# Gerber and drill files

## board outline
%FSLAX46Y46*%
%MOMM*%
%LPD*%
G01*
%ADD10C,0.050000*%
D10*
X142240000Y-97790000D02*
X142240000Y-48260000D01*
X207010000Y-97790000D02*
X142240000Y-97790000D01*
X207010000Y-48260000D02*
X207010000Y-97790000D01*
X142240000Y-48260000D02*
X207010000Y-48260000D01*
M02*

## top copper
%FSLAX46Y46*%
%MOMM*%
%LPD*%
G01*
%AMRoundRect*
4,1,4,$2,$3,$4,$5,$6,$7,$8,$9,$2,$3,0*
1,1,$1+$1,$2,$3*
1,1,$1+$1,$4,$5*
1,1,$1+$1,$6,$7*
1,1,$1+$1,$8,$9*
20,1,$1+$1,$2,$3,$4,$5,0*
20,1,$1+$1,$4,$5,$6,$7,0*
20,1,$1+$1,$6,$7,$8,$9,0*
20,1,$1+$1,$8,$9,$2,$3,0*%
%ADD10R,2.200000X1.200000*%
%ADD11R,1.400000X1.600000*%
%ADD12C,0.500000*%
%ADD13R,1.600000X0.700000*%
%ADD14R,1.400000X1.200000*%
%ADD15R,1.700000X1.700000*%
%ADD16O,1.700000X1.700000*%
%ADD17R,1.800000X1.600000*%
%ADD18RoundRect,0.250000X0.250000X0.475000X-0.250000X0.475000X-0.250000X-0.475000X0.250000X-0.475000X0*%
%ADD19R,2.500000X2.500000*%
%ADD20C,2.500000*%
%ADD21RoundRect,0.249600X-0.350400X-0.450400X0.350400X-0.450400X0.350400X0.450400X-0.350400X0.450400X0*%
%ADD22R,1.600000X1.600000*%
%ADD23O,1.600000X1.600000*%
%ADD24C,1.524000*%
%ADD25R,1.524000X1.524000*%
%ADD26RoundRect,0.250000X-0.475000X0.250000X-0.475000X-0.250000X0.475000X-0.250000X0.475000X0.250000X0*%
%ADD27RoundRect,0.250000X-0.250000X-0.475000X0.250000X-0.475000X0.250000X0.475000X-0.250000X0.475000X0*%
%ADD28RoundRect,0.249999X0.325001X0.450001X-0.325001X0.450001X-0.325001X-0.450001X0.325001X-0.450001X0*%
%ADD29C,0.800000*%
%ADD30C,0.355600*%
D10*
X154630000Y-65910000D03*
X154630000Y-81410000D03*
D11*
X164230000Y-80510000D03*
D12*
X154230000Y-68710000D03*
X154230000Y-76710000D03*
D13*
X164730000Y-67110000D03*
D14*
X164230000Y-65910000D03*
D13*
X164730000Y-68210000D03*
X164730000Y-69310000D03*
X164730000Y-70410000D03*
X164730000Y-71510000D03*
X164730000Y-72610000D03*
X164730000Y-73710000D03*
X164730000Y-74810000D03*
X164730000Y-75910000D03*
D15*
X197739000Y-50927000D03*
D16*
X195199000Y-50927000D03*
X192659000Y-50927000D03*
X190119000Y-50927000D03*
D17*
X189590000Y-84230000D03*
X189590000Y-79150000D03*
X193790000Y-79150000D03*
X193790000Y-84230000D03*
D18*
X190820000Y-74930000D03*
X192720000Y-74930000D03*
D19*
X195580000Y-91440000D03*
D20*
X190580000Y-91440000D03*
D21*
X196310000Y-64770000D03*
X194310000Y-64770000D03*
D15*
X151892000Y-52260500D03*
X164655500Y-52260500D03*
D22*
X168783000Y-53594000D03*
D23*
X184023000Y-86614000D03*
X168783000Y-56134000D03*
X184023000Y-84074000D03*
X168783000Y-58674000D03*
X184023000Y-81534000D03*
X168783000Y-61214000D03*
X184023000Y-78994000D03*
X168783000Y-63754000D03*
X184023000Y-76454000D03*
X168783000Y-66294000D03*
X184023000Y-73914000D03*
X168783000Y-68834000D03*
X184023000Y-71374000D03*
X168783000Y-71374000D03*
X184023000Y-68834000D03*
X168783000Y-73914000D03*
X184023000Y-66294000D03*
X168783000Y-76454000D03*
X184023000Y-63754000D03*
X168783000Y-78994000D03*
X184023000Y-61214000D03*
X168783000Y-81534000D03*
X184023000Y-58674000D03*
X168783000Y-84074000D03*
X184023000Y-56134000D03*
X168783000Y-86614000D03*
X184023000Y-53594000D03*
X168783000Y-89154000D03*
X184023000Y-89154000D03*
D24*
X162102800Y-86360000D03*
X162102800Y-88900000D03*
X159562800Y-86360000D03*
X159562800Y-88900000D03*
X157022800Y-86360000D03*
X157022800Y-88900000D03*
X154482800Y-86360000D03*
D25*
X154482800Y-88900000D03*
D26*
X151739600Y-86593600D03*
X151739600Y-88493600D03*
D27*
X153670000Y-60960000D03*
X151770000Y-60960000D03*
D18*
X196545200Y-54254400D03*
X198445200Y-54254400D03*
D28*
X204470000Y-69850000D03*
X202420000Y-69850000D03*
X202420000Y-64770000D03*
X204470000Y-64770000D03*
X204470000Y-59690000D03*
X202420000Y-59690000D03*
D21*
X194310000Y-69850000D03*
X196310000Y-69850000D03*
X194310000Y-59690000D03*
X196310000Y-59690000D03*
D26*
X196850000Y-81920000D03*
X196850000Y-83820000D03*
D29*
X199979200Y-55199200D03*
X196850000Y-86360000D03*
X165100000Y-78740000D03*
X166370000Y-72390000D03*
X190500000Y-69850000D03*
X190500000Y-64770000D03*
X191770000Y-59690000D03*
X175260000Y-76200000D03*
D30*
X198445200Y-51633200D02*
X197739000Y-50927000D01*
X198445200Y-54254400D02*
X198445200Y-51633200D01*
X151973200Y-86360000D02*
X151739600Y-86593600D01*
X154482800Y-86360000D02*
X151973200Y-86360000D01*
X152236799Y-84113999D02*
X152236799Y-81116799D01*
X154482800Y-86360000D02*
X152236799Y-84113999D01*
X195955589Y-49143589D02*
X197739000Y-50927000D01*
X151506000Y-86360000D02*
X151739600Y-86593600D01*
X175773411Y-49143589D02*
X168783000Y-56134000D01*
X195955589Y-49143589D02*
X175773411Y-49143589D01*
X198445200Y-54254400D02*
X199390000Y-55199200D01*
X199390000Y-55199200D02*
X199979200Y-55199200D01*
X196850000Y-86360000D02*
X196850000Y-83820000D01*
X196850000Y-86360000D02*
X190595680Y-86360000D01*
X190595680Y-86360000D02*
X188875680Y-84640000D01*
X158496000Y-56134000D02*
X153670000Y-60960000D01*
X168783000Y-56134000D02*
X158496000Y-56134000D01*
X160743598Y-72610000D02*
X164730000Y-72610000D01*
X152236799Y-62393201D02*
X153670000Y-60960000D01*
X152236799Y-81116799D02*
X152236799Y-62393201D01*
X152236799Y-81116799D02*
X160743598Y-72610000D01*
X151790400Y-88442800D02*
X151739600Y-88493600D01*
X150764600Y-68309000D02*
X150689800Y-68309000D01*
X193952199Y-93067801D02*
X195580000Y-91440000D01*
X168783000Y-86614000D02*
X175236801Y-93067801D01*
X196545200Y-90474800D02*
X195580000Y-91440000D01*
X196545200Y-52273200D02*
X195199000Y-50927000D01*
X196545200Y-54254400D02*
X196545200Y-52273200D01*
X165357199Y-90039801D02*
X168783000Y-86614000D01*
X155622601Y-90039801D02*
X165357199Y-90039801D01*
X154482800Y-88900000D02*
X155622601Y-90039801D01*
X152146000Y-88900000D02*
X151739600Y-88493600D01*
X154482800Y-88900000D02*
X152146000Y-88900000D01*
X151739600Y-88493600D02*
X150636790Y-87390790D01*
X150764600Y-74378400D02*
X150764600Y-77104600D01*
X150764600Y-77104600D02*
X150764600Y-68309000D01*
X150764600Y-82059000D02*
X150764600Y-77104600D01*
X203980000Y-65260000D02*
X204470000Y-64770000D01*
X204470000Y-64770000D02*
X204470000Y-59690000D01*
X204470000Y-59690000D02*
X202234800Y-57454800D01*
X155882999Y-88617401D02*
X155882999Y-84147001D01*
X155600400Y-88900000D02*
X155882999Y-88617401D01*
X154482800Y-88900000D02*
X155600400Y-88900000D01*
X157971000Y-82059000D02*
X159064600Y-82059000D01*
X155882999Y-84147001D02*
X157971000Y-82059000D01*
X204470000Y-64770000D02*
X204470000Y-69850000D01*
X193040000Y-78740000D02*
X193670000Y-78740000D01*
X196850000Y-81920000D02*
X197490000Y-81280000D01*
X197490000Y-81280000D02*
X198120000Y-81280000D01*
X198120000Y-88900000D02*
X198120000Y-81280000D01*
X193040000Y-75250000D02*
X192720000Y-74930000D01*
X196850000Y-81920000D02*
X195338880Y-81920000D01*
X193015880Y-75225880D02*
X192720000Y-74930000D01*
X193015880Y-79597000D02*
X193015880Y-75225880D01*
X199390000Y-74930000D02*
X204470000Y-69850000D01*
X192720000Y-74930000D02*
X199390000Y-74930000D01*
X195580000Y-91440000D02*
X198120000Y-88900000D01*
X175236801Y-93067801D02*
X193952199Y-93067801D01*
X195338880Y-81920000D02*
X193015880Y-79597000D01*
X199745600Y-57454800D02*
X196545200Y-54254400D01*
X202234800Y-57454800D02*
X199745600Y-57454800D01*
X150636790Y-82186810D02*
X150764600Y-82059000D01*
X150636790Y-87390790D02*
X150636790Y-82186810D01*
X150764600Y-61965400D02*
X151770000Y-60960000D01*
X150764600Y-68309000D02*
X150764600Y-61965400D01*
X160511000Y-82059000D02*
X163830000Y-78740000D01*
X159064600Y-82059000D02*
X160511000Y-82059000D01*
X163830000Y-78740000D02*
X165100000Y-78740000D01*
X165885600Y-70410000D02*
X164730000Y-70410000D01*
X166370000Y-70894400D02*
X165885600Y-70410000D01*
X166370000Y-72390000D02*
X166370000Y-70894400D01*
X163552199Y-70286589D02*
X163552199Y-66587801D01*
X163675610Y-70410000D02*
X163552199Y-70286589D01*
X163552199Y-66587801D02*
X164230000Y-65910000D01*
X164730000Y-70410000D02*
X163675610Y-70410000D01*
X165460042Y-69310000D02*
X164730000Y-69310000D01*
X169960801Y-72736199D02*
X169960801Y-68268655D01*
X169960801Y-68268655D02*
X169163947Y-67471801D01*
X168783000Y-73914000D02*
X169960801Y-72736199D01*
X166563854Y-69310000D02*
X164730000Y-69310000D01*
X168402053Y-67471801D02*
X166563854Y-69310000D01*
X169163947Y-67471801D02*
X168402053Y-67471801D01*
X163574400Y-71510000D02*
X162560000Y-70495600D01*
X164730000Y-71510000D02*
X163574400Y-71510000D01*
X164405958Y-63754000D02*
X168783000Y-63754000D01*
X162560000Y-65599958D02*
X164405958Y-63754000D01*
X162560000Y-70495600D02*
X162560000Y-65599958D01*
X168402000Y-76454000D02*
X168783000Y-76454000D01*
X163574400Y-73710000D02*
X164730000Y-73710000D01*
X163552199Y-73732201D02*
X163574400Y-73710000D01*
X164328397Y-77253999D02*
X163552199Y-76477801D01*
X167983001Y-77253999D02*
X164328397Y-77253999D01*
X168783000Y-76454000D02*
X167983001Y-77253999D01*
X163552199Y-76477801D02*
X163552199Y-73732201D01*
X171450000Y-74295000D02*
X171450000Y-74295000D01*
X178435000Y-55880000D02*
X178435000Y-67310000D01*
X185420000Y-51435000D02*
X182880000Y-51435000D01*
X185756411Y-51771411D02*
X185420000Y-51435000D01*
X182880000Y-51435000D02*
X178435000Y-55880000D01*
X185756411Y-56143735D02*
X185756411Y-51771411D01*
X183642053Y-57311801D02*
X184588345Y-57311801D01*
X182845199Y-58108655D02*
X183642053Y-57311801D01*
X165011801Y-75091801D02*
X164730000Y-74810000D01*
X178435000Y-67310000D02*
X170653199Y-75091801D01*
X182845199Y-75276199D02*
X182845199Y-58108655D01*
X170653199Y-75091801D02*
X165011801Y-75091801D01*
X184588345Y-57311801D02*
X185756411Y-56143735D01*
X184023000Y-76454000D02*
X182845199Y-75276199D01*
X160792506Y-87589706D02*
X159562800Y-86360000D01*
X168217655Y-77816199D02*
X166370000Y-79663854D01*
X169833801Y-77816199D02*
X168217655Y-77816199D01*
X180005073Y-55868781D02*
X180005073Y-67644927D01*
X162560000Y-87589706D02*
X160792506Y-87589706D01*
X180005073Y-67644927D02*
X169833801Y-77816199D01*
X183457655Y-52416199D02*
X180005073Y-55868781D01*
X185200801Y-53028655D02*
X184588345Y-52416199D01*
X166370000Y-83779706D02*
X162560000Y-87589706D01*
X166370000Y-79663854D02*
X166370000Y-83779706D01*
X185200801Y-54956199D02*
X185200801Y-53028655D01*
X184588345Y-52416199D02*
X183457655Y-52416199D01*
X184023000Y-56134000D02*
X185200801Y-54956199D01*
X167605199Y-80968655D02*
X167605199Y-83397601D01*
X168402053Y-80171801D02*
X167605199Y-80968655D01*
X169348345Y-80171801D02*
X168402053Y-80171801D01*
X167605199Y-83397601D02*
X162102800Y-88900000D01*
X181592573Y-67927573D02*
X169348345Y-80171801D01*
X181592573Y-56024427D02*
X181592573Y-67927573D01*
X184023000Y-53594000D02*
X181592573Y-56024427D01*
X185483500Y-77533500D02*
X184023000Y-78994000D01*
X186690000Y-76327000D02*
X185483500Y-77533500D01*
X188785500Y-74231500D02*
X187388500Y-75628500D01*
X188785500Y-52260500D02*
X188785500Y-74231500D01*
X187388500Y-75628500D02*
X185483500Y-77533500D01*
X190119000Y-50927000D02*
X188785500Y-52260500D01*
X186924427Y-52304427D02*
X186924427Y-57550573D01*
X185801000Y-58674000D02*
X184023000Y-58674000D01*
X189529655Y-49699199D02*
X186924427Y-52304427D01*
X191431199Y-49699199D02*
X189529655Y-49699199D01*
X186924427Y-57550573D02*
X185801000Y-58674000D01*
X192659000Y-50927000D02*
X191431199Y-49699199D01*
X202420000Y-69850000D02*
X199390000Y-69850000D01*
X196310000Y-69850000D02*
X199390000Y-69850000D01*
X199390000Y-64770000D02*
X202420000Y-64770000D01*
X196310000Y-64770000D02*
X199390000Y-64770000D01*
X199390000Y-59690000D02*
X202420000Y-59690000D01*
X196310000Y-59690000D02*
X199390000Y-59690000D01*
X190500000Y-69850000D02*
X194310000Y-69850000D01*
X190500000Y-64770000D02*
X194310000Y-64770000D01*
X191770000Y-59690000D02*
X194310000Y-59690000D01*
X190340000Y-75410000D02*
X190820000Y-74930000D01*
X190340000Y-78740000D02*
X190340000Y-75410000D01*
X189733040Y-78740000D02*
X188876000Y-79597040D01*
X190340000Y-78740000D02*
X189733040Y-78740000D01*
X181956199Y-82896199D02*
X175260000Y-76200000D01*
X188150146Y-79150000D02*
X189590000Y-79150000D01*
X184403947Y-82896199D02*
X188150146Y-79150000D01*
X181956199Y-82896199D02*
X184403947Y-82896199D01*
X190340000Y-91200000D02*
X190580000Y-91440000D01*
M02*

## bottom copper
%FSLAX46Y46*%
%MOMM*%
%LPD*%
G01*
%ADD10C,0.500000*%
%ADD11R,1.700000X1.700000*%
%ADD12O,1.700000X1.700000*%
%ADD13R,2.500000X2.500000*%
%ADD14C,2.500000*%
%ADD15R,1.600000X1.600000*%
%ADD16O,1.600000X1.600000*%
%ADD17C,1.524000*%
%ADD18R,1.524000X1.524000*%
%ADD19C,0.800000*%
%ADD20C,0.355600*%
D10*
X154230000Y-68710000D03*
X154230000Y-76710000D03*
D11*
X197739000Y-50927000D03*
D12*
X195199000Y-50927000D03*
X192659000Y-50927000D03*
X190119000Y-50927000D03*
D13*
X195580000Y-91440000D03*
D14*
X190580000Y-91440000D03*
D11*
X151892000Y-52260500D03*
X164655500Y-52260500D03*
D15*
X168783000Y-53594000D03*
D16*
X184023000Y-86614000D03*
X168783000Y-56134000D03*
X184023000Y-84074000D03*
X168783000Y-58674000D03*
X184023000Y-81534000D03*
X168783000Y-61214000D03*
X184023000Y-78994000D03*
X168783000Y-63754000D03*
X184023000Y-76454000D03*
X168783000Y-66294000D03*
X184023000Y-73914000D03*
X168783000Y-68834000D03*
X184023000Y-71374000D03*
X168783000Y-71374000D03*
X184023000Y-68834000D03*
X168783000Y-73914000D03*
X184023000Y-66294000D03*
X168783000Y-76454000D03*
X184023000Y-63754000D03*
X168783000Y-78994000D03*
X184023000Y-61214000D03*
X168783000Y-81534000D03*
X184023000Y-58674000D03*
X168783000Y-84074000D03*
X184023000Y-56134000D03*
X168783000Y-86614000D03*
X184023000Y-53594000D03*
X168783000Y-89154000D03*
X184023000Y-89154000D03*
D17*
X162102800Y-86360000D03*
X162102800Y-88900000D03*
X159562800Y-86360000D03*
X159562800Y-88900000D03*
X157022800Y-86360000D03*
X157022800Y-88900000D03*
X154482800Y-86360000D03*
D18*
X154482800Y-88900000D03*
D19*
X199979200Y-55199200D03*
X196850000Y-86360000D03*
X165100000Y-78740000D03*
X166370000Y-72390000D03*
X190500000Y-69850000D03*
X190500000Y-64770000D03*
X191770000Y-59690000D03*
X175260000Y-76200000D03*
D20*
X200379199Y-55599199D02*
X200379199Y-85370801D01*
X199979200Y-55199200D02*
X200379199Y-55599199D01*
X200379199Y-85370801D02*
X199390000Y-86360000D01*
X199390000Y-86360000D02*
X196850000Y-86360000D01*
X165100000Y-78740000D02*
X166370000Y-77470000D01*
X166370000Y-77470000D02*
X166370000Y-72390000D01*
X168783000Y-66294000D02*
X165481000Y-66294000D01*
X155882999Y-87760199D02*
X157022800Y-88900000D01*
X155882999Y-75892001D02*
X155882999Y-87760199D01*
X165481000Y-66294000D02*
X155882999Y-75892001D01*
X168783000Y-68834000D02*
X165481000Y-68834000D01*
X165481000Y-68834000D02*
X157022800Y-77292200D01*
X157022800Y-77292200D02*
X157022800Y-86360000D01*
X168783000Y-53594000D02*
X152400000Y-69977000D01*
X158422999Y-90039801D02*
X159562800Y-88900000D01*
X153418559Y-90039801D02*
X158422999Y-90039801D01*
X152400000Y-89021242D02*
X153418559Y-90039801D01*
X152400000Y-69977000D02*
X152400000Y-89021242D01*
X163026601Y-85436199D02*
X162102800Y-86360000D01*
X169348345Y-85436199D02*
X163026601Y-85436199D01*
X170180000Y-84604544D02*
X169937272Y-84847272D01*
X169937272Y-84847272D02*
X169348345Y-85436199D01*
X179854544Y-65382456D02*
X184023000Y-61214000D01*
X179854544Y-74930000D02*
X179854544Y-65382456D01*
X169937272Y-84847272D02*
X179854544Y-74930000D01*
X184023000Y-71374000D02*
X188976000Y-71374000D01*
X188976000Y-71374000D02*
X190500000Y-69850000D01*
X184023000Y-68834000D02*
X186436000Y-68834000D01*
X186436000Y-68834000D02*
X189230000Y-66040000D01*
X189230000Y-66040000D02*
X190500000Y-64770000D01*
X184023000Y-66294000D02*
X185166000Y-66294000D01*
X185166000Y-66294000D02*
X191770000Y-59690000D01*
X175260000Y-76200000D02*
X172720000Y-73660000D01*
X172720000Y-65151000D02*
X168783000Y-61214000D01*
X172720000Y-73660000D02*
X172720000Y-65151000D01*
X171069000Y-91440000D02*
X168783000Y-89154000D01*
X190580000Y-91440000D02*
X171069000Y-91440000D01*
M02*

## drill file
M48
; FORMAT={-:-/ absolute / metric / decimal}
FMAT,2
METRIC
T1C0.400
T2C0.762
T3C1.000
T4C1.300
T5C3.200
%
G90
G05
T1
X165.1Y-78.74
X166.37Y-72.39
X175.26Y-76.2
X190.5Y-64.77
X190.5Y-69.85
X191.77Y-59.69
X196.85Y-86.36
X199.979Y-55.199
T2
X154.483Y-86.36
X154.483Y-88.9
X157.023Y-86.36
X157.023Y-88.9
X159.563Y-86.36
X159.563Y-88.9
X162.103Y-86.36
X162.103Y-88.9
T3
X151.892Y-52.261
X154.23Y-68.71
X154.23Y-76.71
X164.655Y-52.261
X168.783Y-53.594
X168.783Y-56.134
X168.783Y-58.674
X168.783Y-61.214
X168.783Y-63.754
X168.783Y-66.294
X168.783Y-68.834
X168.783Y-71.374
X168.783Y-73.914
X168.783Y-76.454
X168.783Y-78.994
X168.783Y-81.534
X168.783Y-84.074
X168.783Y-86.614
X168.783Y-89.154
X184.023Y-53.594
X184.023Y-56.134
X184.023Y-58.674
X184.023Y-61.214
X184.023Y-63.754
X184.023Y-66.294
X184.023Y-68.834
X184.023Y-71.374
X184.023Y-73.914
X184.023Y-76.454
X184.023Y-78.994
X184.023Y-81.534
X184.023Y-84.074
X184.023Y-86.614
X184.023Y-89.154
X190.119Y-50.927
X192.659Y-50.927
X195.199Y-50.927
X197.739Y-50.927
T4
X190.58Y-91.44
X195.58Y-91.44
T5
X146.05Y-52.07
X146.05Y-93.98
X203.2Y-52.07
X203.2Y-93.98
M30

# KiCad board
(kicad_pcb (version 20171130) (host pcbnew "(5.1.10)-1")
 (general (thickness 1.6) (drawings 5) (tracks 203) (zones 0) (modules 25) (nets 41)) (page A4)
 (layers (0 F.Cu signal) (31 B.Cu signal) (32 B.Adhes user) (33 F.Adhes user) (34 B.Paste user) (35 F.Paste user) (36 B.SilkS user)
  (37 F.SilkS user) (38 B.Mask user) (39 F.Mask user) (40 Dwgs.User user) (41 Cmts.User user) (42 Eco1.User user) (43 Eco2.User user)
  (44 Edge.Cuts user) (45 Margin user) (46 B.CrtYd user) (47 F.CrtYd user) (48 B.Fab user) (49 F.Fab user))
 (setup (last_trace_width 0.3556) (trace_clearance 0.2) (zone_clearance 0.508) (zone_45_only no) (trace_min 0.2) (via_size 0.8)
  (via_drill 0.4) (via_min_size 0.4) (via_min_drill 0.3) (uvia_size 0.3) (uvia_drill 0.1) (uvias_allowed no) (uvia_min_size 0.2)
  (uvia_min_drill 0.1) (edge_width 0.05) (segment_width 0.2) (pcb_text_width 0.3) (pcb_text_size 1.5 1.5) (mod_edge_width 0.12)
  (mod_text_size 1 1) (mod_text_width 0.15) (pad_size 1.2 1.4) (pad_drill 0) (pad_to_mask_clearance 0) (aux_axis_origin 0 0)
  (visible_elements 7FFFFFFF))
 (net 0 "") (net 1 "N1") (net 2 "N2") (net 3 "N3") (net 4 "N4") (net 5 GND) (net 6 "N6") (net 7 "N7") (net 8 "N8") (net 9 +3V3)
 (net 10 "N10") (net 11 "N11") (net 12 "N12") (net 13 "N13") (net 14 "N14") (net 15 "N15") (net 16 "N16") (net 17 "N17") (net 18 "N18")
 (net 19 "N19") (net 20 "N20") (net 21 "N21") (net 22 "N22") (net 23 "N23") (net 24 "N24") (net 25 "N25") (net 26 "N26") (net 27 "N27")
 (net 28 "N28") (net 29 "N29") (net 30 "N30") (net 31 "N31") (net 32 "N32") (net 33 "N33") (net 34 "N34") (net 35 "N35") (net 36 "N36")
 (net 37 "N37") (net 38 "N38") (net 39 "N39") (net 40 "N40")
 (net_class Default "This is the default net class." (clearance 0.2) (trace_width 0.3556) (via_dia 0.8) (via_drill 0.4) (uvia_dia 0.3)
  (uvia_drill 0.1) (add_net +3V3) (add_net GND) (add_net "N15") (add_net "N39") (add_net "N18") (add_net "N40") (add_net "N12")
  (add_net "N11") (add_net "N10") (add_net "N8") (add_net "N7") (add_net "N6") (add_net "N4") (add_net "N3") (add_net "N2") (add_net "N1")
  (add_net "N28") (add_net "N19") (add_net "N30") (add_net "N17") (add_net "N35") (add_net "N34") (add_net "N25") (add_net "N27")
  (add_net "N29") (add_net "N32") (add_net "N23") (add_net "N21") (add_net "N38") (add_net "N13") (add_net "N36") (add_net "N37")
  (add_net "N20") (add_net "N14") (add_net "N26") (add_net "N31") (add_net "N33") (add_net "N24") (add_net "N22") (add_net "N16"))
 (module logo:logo (layer B.Cu) (at 203.2 68.58 270)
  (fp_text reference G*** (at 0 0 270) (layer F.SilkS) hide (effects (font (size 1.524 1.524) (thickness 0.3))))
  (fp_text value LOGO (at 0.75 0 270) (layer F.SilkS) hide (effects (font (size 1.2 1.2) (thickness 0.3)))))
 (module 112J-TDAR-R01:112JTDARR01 (layer F.Cu) (at 157.48 73.66 270)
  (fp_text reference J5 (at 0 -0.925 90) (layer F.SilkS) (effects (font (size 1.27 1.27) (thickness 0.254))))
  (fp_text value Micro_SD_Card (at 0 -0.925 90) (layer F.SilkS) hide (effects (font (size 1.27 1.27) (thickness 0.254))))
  (pad MP3 smd rect (at -7.75 2.85 270) (size 1.2 2.2) (layers F.Cu F.Paste F.Mask) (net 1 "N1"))
  (pad MP2 smd rect (at 7.75 2.85 270) (size 1.2 2.2) (layers F.Cu F.Paste F.Mask) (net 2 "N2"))
  (pad MP1 smd rect (at 6.85 -6.75) (size 1.4 1.6) (layers F.Cu F.Paste F.Mask) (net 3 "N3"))
  (pad MH2 thru_hole circle (at -4.95 3.25) (size 0.5 0.5) (drill 1) (layers *.Cu *.Mask F.SilkS))
  (pad MH1 thru_hole circle (at 3.05 3.25) (size 0.5 0.5) (drill 1) (layers *.Cu *.Mask F.SilkS))
  (pad CD1 smd rect (at -6.55 -7.25 270) (size 0.7 1.6) (layers F.Cu F.Paste F.Mask) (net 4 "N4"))
  (pad G1 smd rect (at -7.75 -6.75 270) (size 1.2 1.4) (layers F.Cu F.Paste F.Mask) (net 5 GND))
  (pad 8 smd rect (at -5.45 -7.25 270) (size 0.7 1.6) (layers F.Cu F.Paste F.Mask) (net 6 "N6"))
  (pad 7 smd rect (at -4.35 -7.25 270) (size 0.7 1.6) (layers F.Cu F.Paste F.Mask) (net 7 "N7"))
  (pad 6 smd rect (at -3.25 -7.25 270) (size 0.7 1.6) (layers F.Cu F.Paste F.Mask) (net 5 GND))
  (pad 5 smd rect (at -2.15 -7.25 270) (size 0.7 1.6) (layers F.Cu F.Paste F.Mask) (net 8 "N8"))
  (pad 4 smd rect (at -1.05 -7.25 270) (size 0.7 1.6) (layers F.Cu F.Paste F.Mask) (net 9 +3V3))
  (pad 3 smd rect (at 0.05 -7.25 270) (size 0.7 1.6) (layers F.Cu F.Paste F.Mask) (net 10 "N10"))
  (pad 2 smd rect (at 1.15 -7.25 270) (size 0.7 1.6) (layers F.Cu F.Paste F.Mask) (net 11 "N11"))
  (pad 1 smd rect (at 2.25 -7.25 270) (size 0.7 1.6) (layers F.Cu F.Paste F.Mask) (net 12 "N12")))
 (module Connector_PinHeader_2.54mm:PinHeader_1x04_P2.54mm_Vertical (layer F.Cu) (at 197.739 50.927 270)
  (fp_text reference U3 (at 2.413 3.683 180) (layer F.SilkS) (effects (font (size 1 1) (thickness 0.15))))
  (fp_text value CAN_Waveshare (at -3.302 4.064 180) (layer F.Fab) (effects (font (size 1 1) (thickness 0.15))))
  (pad 3.3V thru_hole rect (at 0 0 270) (size 1.7 1.7) (drill 1) (layers *.Cu *.Mask) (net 9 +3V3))
  (pad GND thru_hole oval (at 0 2.54 270) (size 1.7 1.7) (drill 1) (layers *.Cu *.Mask) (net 5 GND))
  (pad CAN_RX thru_hole oval (at 0 5.08 270) (size 1.7 1.7) (drill 1) (layers *.Cu *.Mask) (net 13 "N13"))
  (pad CAN_TX thru_hole oval (at 0 7.62 270) (size 1.7 1.7) (drill 1) (layers *.Cu *.Mask) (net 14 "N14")))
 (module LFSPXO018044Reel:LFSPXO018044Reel (layer F.Cu) (at 191.69 81.69 90)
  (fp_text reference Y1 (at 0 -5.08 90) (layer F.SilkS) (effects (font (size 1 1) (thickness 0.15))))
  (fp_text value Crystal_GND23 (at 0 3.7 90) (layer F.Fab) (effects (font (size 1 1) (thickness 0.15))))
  (pad 4 smd rect (at -2.54 -2.1 90) (size 1.6 1.8) (layers F.Cu F.Paste F.Mask) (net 9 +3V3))
  (pad 3 smd rect (at 2.54 -2.1 90) (size 1.6 1.8) (layers F.Cu F.Paste F.Mask) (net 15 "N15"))
  (pad 2 smd rect (at 2.54 2.1 90) (size 1.6 1.8) (layers F.Cu F.Paste F.Mask) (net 5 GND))
  (pad 1 smd rect (at -2.54 2.1 90) (size 1.6 1.8) (layers F.Cu F.Paste F.Mask) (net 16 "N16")))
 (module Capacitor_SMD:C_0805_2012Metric (layer F.Cu) (at 191.77 74.93 180)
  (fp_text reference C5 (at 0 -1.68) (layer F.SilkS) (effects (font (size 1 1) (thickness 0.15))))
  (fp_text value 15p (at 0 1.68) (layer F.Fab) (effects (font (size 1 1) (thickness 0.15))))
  (pad 2 smd roundrect (at 0.95 0 180) (size 1 1.45) (layers F.Cu F.Paste F.Mask) (roundrect_rratio 0.25) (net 15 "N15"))
  (pad 1 smd roundrect (at -0.95 0 180) (size 1 1.45) (layers F.Cu F.Paste F.Mask) (roundrect_rratio 0.25) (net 5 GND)))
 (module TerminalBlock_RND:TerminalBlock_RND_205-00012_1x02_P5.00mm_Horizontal (layer F.Cu) (at 195.58 91.44 180)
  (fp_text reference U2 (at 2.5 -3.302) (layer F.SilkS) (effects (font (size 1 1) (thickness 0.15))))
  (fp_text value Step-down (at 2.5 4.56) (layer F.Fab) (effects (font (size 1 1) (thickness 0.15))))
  (pad OUT- thru_hole rect (at 0 0 180) (size 2.5 2.5) (drill 1.3) (layers *.Cu *.Mask) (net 5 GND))
  (pad OUT+ thru_hole circle (at 5 0 180) (size 2.5 2.5) (drill 1.3) (layers *.Cu *.Mask) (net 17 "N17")))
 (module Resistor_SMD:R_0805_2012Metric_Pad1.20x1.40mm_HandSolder (layer F.Cu) (at 195.31 64.77)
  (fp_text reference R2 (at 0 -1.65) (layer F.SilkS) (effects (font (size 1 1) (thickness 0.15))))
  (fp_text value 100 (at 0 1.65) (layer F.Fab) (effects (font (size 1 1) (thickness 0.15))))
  (pad 2 smd roundrect (at 1 0) (size 1.2 1.4) (layers F.Cu F.Paste F.Mask) (roundrect_rratio 0.208) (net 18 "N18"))
  (pad 1 smd roundrect (at -1 0) (size 1.2 1.4) (layers F.Cu F.Paste F.Mask) (roundrect_rratio 0.208) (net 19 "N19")))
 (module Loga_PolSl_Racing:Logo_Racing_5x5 (layer B.Cu) (at 146.05 60.96 270)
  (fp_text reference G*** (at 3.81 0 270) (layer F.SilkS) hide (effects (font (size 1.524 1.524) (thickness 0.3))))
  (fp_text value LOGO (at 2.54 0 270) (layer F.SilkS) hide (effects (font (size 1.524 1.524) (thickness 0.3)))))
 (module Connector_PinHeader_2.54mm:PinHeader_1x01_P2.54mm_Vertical (layer F.Cu) (at 151.892 52.2605)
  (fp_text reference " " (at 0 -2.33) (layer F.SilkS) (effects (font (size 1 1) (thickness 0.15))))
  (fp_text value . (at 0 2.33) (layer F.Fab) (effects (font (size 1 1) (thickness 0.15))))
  (pad 1 thru_hole rect (at 0 0) (size 1.7 1.7) (drill 1) (layers *.Cu *.Mask)))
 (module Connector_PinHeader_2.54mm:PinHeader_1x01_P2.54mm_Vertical (layer F.Cu) (at 164.6555 52.2605)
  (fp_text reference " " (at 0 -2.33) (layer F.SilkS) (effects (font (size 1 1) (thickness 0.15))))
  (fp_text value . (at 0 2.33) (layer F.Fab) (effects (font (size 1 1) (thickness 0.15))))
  (pad 1 thru_hole rect (at 0 0) (size 1.7 1.7) (drill 1) (layers *.Cu *.Mask)))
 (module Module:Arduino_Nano (layer F.Cu) (at 168.783 53.594)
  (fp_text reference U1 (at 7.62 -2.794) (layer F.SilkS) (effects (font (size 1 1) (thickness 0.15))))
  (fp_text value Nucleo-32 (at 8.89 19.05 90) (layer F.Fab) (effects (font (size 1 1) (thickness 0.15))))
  (pad D13 thru_hole rect (at 0 0) (size 1.6 1.6) (drill 1) (layers *.Cu *.Mask) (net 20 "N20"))
  (pad D0 thru_hole oval (at 15.24 33.02) (size 1.6 1.6) (drill 1) (layers *.Cu *.Mask) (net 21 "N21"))
  (pad 14 thru_hole oval (at 0 2.54) (size 1.6 1.6) (drill 1) (layers *.Cu *.Mask) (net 9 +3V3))
  (pad NRST thru_hole oval (at 15.24 30.48) (size 1.6 1.6) (drill 1) (layers *.Cu *.Mask) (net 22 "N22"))
  (pad AREF thru_hole oval (at 0 5.08) (size 1.6 1.6) (drill 1) (layers *.Cu *.Mask) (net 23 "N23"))
  (pad GND thru_hole oval (at 15.24 27.94) (size 1.6 1.6) (drill 1) (layers *.Cu *.Mask) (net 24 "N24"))
  (pad A0 thru_hole oval (at 0 7.62) (size 1.6 1.6) (drill 1) (layers *.Cu *.Mask) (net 15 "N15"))
  (pad D2 thru_hole oval (at 15.24 25.4) (size 1.6 1.6) (drill 1) (layers *.Cu *.Mask) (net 14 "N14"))
  (pad A1 thru_hole oval (at 0 10.16) (size 1.6 1.6) (drill 1) (layers *.Cu *.Mask) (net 8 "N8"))
  (pad D3 thru_hole oval (at 15.24 22.86) (size 1.6 1.6) (drill 1) (layers *.Cu *.Mask) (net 11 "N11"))
  (pad A2 thru_hole oval (at 0 12.7) (size 1.6 1.6) (drill 1) (layers *.Cu *.Mask) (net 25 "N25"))
  (pad D4 thru_hole oval (at 15.24 20.32) (size 1.6 1.6) (drill 1) (layers *.Cu *.Mask) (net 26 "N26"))
  (pad A3 thru_hole oval (at 0 15.24) (size 1.6 1.6) (drill 1) (layers *.Cu *.Mask) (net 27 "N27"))
  (pad D5 thru_hole oval (at 15.24 17.78) (size 1.6 1.6) (drill 1) (layers *.Cu *.Mask) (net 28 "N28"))
  (pad A4 thru_hole oval (at 0 17.78) (size 1.6 1.6) (drill 1) (layers *.Cu *.Mask) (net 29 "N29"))
  (pad D6 thru_hole oval (at 15.24 15.24) (size 1.6 1.6) (drill 1) (layers *.Cu *.Mask) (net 19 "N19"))
  (pad A5 thru_hole oval (at 0 20.32) (size 1.6 1.6) (drill 1) (layers *.Cu *.Mask) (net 7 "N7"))
  (pad D7 thru_hole oval (at 15.24 12.7) (size 1.6 1.6) (drill 1) (layers *.Cu *.Mask) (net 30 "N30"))
  (pad A6 thru_hole oval (at 0 22.86) (size 1.6 1.6) (drill 1) (layers *.Cu *.Mask) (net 10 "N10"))
  (pad D8 thru_hole oval (at 15.24 10.16) (size 1.6 1.6) (drill 1) (layers *.Cu *.Mask) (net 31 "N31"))
  (pad A7 thru_hole oval (at 0 25.4) (size 1.6 1.6) (drill 1) (layers *.Cu *.Mask) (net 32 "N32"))
  (pad D9 thru_hole oval (at 15.24 7.62) (size 1.6 1.6) (drill 1) (layers *.Cu *.Mask) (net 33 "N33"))
  (pad 4 thru_hole oval (at 0 27.94) (size 1.6 1.6) (drill 1) (layers *.Cu *.Mask) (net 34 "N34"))
  (pad D10 thru_hole oval (at 15.24 5.08) (size 1.6 1.6) (drill 1) (layers *.Cu *.Mask) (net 13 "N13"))
  (pad 3 thru_hole oval (at 0 30.48) (size 1.6 1.6) (drill 1) (layers *.Cu *.Mask) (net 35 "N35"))
  (pad D11 thru_hole oval (at 15.24 2.54) (size 1.6 1.6) (drill 1) (layers *.Cu *.Mask) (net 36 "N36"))
  (pad 2 thru_hole oval (at 0 33.02) (size 1.6 1.6) (drill 1) (layers *.Cu *.Mask) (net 5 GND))
  (pad D12 thru_hole oval (at 15.24 0) (size 1.6 1.6) (drill 1) (layers *.Cu *.Mask) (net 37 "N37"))
  (pad 1 thru_hole oval (at 0 35.56) (size 1.6 1.6) (drill 1) (layers *.Cu *.Mask) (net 17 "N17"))
  (pad D1 thru_hole oval (at 15.24 35.56) (size 1.6 1.6) (drill 1) (layers *.Cu *.Mask) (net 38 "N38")))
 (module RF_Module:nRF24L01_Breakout (layer F.Cu) (at 152.5778 88.9 90)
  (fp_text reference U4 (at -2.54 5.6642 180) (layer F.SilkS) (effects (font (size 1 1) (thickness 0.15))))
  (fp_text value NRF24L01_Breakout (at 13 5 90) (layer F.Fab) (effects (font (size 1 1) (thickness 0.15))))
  (pad 8 thru_hole circle (at 2.54 9.525 90) (size 1.524 1.524) (drill 0.762) (layers *.Cu *.Mask) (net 33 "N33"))
  (pad 7 thru_hole circle (at 0 9.525 90) (size 1.524 1.524) (drill 0.762) (layers *.Cu *.Mask) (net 37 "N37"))
  (pad 6 thru_hole circle (at 2.54 6.985 90) (size 1.524 1.524) (drill 0.762) (layers *.Cu *.Mask) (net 36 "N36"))
  (pad 5 thru_hole circle (at 0 6.985 90) (size 1.524 1.524) (drill 0.762) (layers *.Cu *.Mask) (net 20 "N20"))
  (pad 4 thru_hole circle (at 2.54 4.445 90) (size 1.524 1.524) (drill 0.762) (layers *.Cu *.Mask) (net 27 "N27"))
  (pad 3 thru_hole circle (at 0 4.445 90) (size 1.524 1.524) (drill 0.762) (layers *.Cu *.Mask) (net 25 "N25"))
  (pad 2 thru_hole circle (at 2.54 1.905 90) (size 1.524 1.524) (drill 0.762) (layers *.Cu *.Mask) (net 9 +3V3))
  (pad 1 thru_hole rect (at 0 1.905 90) (size 1.524 1.524) (drill 0.762) (layers *.Cu *.Mask) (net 5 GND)))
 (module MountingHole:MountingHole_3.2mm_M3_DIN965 (layer F.Cu) (at 146.05 52.07)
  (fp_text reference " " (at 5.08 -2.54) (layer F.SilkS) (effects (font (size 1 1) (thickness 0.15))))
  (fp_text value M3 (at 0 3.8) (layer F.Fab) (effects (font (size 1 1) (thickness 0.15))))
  (pad 1 np_thru_hole circle (at 0 0) (size 3.2 3.2) (drill 3.2) (layers *.Cu *.Mask)))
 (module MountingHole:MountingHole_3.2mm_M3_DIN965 (layer F.Cu) (at 203.2 52.07)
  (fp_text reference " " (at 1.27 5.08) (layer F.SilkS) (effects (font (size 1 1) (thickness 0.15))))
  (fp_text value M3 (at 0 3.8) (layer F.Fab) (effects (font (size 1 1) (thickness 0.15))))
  (pad 1 np_thru_hole circle (at 0 0) (size 3.2 3.2) (drill 3.2) (layers *.Cu *.Mask)))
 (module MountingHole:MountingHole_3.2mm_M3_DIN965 (layer F.Cu) (at 203.2 93.98)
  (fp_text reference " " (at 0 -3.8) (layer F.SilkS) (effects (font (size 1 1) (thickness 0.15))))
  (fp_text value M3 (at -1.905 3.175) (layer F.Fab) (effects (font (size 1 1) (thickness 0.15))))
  (pad 1 np_thru_hole circle (at 0 0) (size 3.2 3.2) (drill 3.2) (layers *.Cu *.Mask)))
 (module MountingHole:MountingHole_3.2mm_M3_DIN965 (layer F.Cu) (at 146.05 93.98)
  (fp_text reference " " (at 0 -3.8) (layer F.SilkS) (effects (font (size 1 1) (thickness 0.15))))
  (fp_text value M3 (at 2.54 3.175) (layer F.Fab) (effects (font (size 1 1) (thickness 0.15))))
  (pad 1 np_thru_hole circle (at 0 0) (size 3.2 3.2) (drill 3.2) (layers *.Cu *.Mask)))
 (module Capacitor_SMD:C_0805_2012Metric (layer F.Cu) (at 151.7396 87.5436 270)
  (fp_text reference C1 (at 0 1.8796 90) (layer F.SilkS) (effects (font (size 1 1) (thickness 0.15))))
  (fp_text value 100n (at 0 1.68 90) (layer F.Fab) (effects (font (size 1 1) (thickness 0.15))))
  (pad 1 smd roundrect (at -0.95 0 270) (size 1 1.45) (layers F.Cu F.Paste F.Mask) (roundrect_rratio 0.25) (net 9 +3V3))
  (pad 2 smd roundrect (at 0.95 0 270) (size 1 1.45) (layers F.Cu F.Paste F.Mask) (roundrect_rratio 0.25) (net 5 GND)))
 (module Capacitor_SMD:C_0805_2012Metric (layer F.Cu) (at 152.72 60.96)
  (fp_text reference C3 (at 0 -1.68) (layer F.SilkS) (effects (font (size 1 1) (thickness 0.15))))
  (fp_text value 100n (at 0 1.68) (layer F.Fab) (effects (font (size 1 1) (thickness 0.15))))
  (pad 2 smd roundrect (at 0.95 0) (size 1 1.45) (layers F.Cu F.Paste F.Mask) (roundrect_rratio 0.25) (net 9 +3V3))
  (pad 1 smd roundrect (at -0.95 0) (size 1 1.45) (layers F.Cu F.Paste F.Mask) (roundrect_rratio 0.25) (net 5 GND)))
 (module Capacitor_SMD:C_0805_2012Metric (layer F.Cu) (at 197.4952 54.2544 180)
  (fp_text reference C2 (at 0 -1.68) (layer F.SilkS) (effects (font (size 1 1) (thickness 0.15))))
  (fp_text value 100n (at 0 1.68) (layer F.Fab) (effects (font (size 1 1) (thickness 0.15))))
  (pad 2 smd roundrect (at 0.95 0 180) (size 1 1.45) (layers F.Cu F.Paste F.Mask) (roundrect_rratio 0.25) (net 5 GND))
  (pad 1 smd roundrect (at -0.95 0 180) (size 1 1.45) (layers F.Cu F.Paste F.Mask) (roundrect_rratio 0.25) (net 9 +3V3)))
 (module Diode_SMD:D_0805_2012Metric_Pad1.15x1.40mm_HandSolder (layer F.Cu) (at 203.445 69.85 180)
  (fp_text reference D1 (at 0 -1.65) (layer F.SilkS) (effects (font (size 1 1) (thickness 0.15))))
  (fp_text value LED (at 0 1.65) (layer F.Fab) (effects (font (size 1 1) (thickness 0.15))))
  (pad 1 smd roundrect (at -1.025 0 180) (size 1.15 1.4) (layers F.Cu F.Paste F.Mask) (roundrect_rratio 0.2173904347826087) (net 5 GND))
  (pad 2 smd roundrect (at 1.025 0 180) (size 1.15 1.4) (layers F.Cu F.Paste F.Mask) (roundrect_rratio 0.2173904347826087) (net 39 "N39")))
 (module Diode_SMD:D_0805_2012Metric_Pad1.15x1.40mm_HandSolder (layer F.Cu) (at 203.445 64.77 180)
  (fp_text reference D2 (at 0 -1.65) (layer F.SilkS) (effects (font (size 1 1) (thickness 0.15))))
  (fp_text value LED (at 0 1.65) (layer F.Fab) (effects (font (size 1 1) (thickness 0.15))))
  (pad 2 smd roundrect (at 1.025 0 180) (size 1.15 1.4) (layers F.Cu F.Paste F.Mask) (roundrect_rratio 0.2173904347826087) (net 18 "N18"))
  (pad 1 smd roundrect (at -1.025 0 180) (size 1.15 1.4) (layers F.Cu F.Paste F.Mask) (roundrect_rratio 0.2173904347826087) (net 5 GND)))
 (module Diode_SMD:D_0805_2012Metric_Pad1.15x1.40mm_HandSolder (layer F.Cu) (at 203.445 59.69 180)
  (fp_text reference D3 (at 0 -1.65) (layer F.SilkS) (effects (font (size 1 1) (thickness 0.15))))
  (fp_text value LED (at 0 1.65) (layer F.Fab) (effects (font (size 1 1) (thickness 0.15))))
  (pad 1 smd roundrect (at -1.025 0 180) (size 1.15 1.4) (layers F.Cu F.Paste F.Mask) (roundrect_rratio 0.2173904347826087) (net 5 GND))
  (pad 2 smd roundrect (at 1.025 0 180) (size 1.15 1.4) (layers F.Cu F.Paste F.Mask) (roundrect_rratio 0.2173904347826087) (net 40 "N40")))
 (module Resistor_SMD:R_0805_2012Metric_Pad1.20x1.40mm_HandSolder (layer F.Cu) (at 195.31 69.85)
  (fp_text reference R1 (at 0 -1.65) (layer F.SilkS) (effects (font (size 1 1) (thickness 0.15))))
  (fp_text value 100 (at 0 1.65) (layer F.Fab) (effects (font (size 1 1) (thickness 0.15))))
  (pad 1 smd roundrect (at -1 0) (size 1.2 1.4) (layers F.Cu F.Paste F.Mask) (roundrect_rratio 0.208) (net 28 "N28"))
  (pad 2 smd roundrect (at 1 0) (size 1.2 1.4) (layers F.Cu F.Paste F.Mask) (roundrect_rratio 0.208) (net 39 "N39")))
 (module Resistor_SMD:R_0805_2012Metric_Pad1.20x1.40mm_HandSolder (layer F.Cu) (at 195.31 59.69)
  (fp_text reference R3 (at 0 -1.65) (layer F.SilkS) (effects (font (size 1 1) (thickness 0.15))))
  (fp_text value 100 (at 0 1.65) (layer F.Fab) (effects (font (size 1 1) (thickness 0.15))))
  (pad 1 smd roundrect (at -1 0) (size 1.2 1.4) (layers F.Cu F.Paste F.Mask) (roundrect_rratio 0.208) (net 30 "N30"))
  (pad 2 smd roundrect (at 1 0) (size 1.2 1.4) (layers F.Cu F.Paste F.Mask) (roundrect_rratio 0.208) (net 40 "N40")))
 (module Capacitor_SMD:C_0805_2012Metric (layer F.Cu) (at 196.85 82.87 270)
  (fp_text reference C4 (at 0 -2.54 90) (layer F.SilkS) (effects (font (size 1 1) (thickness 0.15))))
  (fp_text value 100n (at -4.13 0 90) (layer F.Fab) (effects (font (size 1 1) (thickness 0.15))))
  (pad 1 smd roundrect (at -0.95 0 270) (size 1 1.45) (layers F.Cu F.Paste F.Mask) (roundrect_rratio 0.25) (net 5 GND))
  (pad 2 smd roundrect (at 0.95 0 270) (size 1 1.45) (layers F.Cu F.Paste F.Mask) (roundrect_rratio 0.25) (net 9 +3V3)))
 (gr_line (start 142.24 97.79) (end 142.24 48.26) (layer Edge.Cuts) (width 0.05))
 (gr_line (start 207.01 97.79) (end 142.24 97.79) (layer Edge.Cuts) (width 0.05))
 (gr_line (start 207.01 48.26) (end 207.01 97.79) (layer Edge.Cuts) (width 0.05))
 (gr_line (start 142.24 48.26) (end 207.01 48.26) (layer Edge.Cuts) (width 0.05))
 (segment (start 198.4452 51.6332) (end 197.739 50.927) (width 0.3556) (layer F.Cu) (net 9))
 (segment (start 198.4452 54.2544) (end 198.4452 51.6332) (width 0.3556) (layer F.Cu) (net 9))
 (segment (start 151.9732 86.36) (end 151.7396 86.5936) (width 0.3556) (layer F.Cu) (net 9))
 (segment (start 154.4828 86.36) (end 151.9732 86.36) (width 0.3556) (layer F.Cu) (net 9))
 (segment (start 152.236799 84.113999) (end 152.236799 81.116799) (width 0.3556) (layer F.Cu) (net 9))
 (segment (start 154.4828 86.36) (end 152.236799 84.113999) (width 0.3556) (layer F.Cu) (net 9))
 (segment (start 195.955589 49.143589) (end 197.739 50.927) (width 0.3556) (layer F.Cu) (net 9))
 (segment (start 151.506 86.36) (end 151.7396 86.5936) (width 0.3556) (layer F.Cu) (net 9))
 (segment (start 175.773411 49.143589) (end 168.783 56.134) (width 0.3556) (layer F.Cu) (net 9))
 (segment (start 195.955589 49.143589) (end 175.773411 49.143589) (width 0.3556) (layer F.Cu) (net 9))
 (segment (start 198.4452 54.2544) (end 199.39 55.1992) (width 0.3556) (layer F.Cu) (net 9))
 (segment (start 199.39 55.1992) (end 199.9792 55.1992) (width 0.3556) (layer F.Cu) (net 9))
 (via (at 199.9792 55.1992) (size 0.8) (drill 0.4) (layers F.Cu B.Cu) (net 9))
 (segment (start 200.379199 55.599199) (end 200.379199 85.370801) (width 0.3556) (layer B.Cu) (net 9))
 (segment (start 199.9792 55.1992) (end 200.379199 55.599199) (width 0.3556) (layer B.Cu) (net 9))
 (segment (start 200.379199 85.370801) (end 199.39 86.36) (width 0.3556) (layer B.Cu) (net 9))
 (via (at 196.85 86.36) (size 0.8) (drill 0.4) (layers F.Cu B.Cu) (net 9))
 (segment (start 199.39 86.36) (end 196.85 86.36) (width 0.3556) (layer B.Cu) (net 9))
 (segment (start 196.85 86.36) (end 196.85 83.82) (width 0.3556) (layer F.Cu) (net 9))
 (segment (start 196.85 86.36) (end 190.59568 86.36) (width 0.3556) (layer F.Cu) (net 9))
 (segment (start 190.59568 86.36) (end 188.87568 84.64) (width 0.3556) (layer F.Cu) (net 9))
 (segment (start 158.496 56.134) (end 153.67 60.96) (width 0.3556) (layer F.Cu) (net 9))
 (segment (start 168.783 56.134) (end 158.496 56.134) (width 0.3556) (layer F.Cu) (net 9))
 (segment (start 160.743598 72.61) (end 164.73 72.61) (width 0.3556) (layer F.Cu) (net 9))
 (segment (start 152.236799 62.393201) (end 153.67 60.96) (width 0.3556) (layer F.Cu) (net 9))
 (segment (start 152.236799 81.116799) (end 152.236799 62.393201) (width 0.3556) (layer F.Cu) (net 9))
 (segment (start 152.236799 81.116799) (end 160.743598 72.61) (width 0.3556) (layer F.Cu) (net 9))
 (segment (start 151.7904 88.4428) (end 151.7396 88.4936) (width 0.3556) (layer F.Cu) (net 5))
 (segment (start 150.7646 68.309) (end 150.6898 68.309) (width 0.3556) (layer F.Cu) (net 5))
 (segment (start 193.952199 93.067801) (end 195.58 91.44) (width 0.3556) (layer F.Cu) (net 5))
 (segment (start 168.783 86.614) (end 175.236801 93.067801) (width 0.3556) (layer F.Cu) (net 5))
 (segment (start 196.5452 90.4748) (end 195.58 91.44) (width 0.3556) (layer F.Cu) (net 5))
 (segment (start 196.5452 52.2732) (end 195.199 50.927) (width 0.3556) (layer F.Cu) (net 5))
 (segment (start 196.5452 54.2544) (end 196.5452 52.2732) (width 0.3556) (layer F.Cu) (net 5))
 (segment (start 165.357199 90.039801) (end 168.783 86.614) (width 0.3556) (layer F.Cu) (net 5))
 (segment (start 155.622601 90.039801) (end 165.357199 90.039801) (width 0.3556) (layer F.Cu) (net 5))
 (segment (start 154.4828 88.9) (end 155.622601 90.039801) (width 0.3556) (layer F.Cu) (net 5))
 (segment (start 152.146 88.9) (end 151.7396 88.4936) (width 0.3556) (layer F.Cu) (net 5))
 (segment (start 154.4828 88.9) (end 152.146 88.9) (width 0.3556) (layer F.Cu) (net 5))
 (segment (start 151.7396 88.4936) (end 150.63679 87.39079) (width 0.3556) (layer F.Cu) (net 5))
 (segment (start 150.7646 74.3784) (end 150.7646 77.1046) (width 0.3556) (layer F.Cu) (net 5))
 (segment (start 150.7646 77.1046) (end 150.7646 68.309) (width 0.3556) (layer F.Cu) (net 5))
 (segment (start 150.7646 82.059) (end 150.7646 77.1046) (width 0.3556) (layer F.Cu) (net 5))
 (segment (start 203.98 65.26) (end 204.47 64.77) (width 0.3556) (layer F.Cu) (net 5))
 (segment (start 204.47 64.77) (end 204.47 59.69) (width 0.3556) (layer F.Cu) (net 5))
 (segment (start 204.47 59.69) (end 202.2348 57.4548) (width 0.3556) (layer F.Cu) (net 5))
 (segment (start 155.882999 88.617401) (end 155.882999 84.147001) (width 0.3556) (layer F.Cu) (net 5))
 (segment (start 155.6004 88.9) (end 155.882999 88.617401) (width 0.3556) (layer F.Cu) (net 5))
 (segment (start 154.4828 88.9) (end 155.6004 88.9) (width 0.3556) (layer F.Cu) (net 5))
 (segment (start 157.971 82.059) (end 159.0646 82.059) (width 0.3556) (layer F.Cu) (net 5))
 (segment (start 155.882999 84.147001) (end 157.971 82.059) (width 0.3556) (layer F.Cu) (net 5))
 (segment (start 204.47 64.77) (end 204.47 69.85) (width 0.3556) (layer F.Cu) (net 5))
 (segment (start 193.04 78.74) (end 193.67 78.74) (width 0.3556) (layer F.Cu) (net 5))
 (segment (start 196.85 81.92) (end 197.49 81.28) (width 0.3556) (layer F.Cu) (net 5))
 (segment (start 197.49 81.28) (end 198.12 81.28) (width 0.3556) (layer F.Cu) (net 5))
 (segment (start 198.12 88.9) (end 198.12 81.28) (width 0.3556) (layer F.Cu) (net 5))
 (segment (start 193.04 75.25) (end 192.72 74.93) (width 0.3556) (layer F.Cu) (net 5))
 (segment (start 196.85 81.92) (end 195.33888 81.92) (width 0.3556) (layer F.Cu) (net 5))
 (segment (start 193.01588 75.22588) (end 192.72 74.93) (width 0.3556) (layer F.Cu) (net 5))
 (segment (start 193.01588 79.597) (end 193.01588 75.22588) (width 0.3556) (layer F.Cu) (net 5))
 (segment (start 199.39 74.93) (end 204.47 69.85) (width 0.3556) (layer F.Cu) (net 5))
 (segment (start 192.72 74.93) (end 199.39 74.93) (width 0.3556) (layer F.Cu) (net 5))
 (segment (start 195.58 91.44) (end 198.12 88.9) (width 0.3556) (layer F.Cu) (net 5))
 (segment (start 175.236801 93.067801) (end 193.952199 93.067801) (width 0.3556) (layer F.Cu) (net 5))
 (segment (start 195.33888 81.92) (end 193.01588 79.597) (width 0.3556) (layer F.Cu) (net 5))
 (segment (start 199.7456 57.4548) (end 196.5452 54.2544) (width 0.3556) (layer F.Cu) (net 5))
 (segment (start 202.2348 57.4548) (end 199.7456 57.4548) (width 0.3556) (layer F.Cu) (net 5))
 (segment (start 150.63679 82.18681) (end 150.7646 82.059) (width 0.3556) (layer F.Cu) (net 5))
 (segment (start 150.63679 87.39079) (end 150.63679 82.18681) (width 0.3556) (layer F.Cu) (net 5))
 (segment (start 150.7646 61.9654) (end 151.77 60.96) (width 0.3556) (layer F.Cu) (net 5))
 (segment (start 150.7646 68.309) (end 150.7646 61.9654) (width 0.3556) (layer F.Cu) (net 5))
 (segment (start 160.511 82.059) (end 163.83 78.74) (width 0.3556) (layer F.Cu) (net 5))
 (segment (start 159.0646 82.059) (end 160.511 82.059) (width 0.3556) (layer F.Cu) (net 5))
 (segment (start 163.83 78.74) (end 165.1 78.74) (width 0.3556) (layer F.Cu) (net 5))
 (via (at 165.1 78.74) (size 0.8) (drill 0.4) (layers F.Cu B.Cu) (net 5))
 (segment (start 165.1 78.74) (end 166.37 77.47) (width 0.3556) (layer B.Cu) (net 5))
 (segment (start 166.37 77.47) (end 166.37 72.39) (width 0.3556) (layer B.Cu) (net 5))
 (via (at 166.37 72.39) (size 0.8) (drill 0.4) (layers F.Cu B.Cu) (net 5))
 (segment (start 165.8856 70.41) (end 164.73 70.41) (width 0.3556) (layer F.Cu) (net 5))
 (segment (start 166.37 70.8944) (end 165.8856 70.41) (width 0.3556) (layer F.Cu) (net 5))
 (segment (start 166.37 72.39) (end 166.37 70.8944) (width 0.3556) (layer F.Cu) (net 5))
 (segment (start 163.552199 70.286589) (end 163.552199 66.587801) (width 0.3556) (layer F.Cu) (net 5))
 (segment (start 163.67561 70.41) (end 163.552199 70.286589) (width 0.3556) (layer F.Cu) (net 5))
 (segment (start 163.552199 66.587801) (end 164.23 65.91) (width 0.3556) (layer F.Cu) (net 5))
 (segment (start 164.73 70.41) (end 163.67561 70.41) (width 0.3556) (layer F.Cu) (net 5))
 (segment (start 165.460042 69.31) (end 164.73 69.31) (width 0.3556) (layer F.Cu) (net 7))
 (segment (start 169.960801 72.736199) (end 169.960801 68.268655) (width 0.3556) (layer F.Cu) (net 7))
 (segment (start 169.960801 68.268655) (end 169.163947 67.471801) (width 0.3556) (layer F.Cu) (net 7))
 (segment (start 168.783 73.914) (end 169.960801 72.736199) (width 0.3556) (layer F.Cu) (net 7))
 (segment (start 166.563854 69.31) (end 164.73 69.31) (width 0.3556) (layer F.Cu) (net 7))
 (segment (start 168.402053 67.471801) (end 166.563854 69.31) (width 0.3556) (layer F.Cu) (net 7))
 (segment (start 169.163947 67.471801) (end 168.402053 67.471801) (width 0.3556) (layer F.Cu) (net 7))
 (segment (start 163.5744 71.51) (end 162.56 70.4956) (width 0.3556) (layer F.Cu) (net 8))
 (segment (start 164.73 71.51) (end 163.5744 71.51) (width 0.3556) (layer F.Cu) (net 8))
 (segment (start 164.405958 63.754) (end 168.783 63.754) (width 0.3556) (layer F.Cu) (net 8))
 (segment (start 162.56 65.599958) (end 164.405958 63.754) (width 0.3556) (layer F.Cu) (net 8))
 (segment (start 162.56 70.4956) (end 162.56 65.599958) (width 0.3556) (layer F.Cu) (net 8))
 (segment (start 168.402 76.454) (end 168.783 76.454) (width 0.3556) (layer F.Cu) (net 10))
 (segment (start 163.5744 73.71) (end 164.73 73.71) (width 0.3556) (layer F.Cu) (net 10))
 (segment (start 163.552199 73.732201) (end 163.5744 73.71) (width 0.3556) (layer F.Cu) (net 10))
 (segment (start 164.328397 77.253999) (end 163.552199 76.477801) (width 0.3556) (layer F.Cu) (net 10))
 (segment (start 167.983001 77.253999) (end 164.328397 77.253999) (width 0.3556) (layer F.Cu) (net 10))
 (segment (start 168.783 76.454) (end 167.983001 77.253999) (width 0.3556) (layer F.Cu) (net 10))
 (segment (start 163.552199 76.477801) (end 163.552199 73.732201) (width 0.3556) (layer F.Cu) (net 10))
 (segment (start 171.45 74.295) (end 171.45 74.295) (width 0.3556) (layer F.Cu) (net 11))
 (segment (start 178.435 55.88) (end 178.435 67.31) (width 0.3556) (layer F.Cu) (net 11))
 (segment (start 185.42 51.435) (end 182.88 51.435) (width 0.3556) (layer F.Cu) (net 11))
 (segment (start 185.756411 51.771411) (end 185.42 51.435) (width 0.3556) (layer F.Cu) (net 11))
 (segment (start 182.88 51.435) (end 178.435 55.88) (width 0.3556) (layer F.Cu) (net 11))
 (segment (start 185.756411 56.143735) (end 185.756411 51.771411) (width 0.3556) (layer F.Cu) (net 11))
 (segment (start 183.642053 57.311801) (end 184.588345 57.311801) (width 0.3556) (layer F.Cu) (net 11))
 (segment (start 182.845199 58.108655) (end 183.642053 57.311801) (width 0.3556) (layer F.Cu) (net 11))
 (segment (start 165.011801 75.091801) (end 164.73 74.81) (width 0.3556) (layer F.Cu) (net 11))
 (segment (start 178.435 67.31) (end 170.653199 75.091801) (width 0.3556) (layer F.Cu) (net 11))
 (segment (start 182.845199 75.276199) (end 182.845199 58.108655) (width 0.3556) (layer F.Cu) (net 11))
 (segment (start 170.653199 75.091801) (end 165.011801 75.091801) (width 0.3556) (layer F.Cu) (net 11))
 (segment (start 184.588345 57.311801) (end 185.756411 56.143735) (width 0.3556) (layer F.Cu) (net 11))
 (segment (start 184.023 76.454) (end 182.845199 75.276199) (width 0.3556) (layer F.Cu) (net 11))
 (segment (start 168.783 66.294) (end 165.481 66.294) (width 0.3556) (layer B.Cu) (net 25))
 (segment (start 155.882999 87.760199) (end 157.0228 88.9) (width 0.3556) (layer B.Cu) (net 25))
 (segment (start 155.882999 75.892001) (end 155.882999 87.760199) (width 0.3556) (layer B.Cu) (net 25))
 (segment (start 165.481 66.294) (end 155.882999 75.892001) (width 0.3556) (layer B.Cu) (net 25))
 (segment (start 168.783 68.834) (end 165.481 68.834) (width 0.3556) (layer B.Cu) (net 27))
 (segment (start 165.481 68.834) (end 157.0228 77.2922) (width 0.3556) (layer B.Cu) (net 27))
 (segment (start 157.0228 77.2922) (end 157.0228 86.36) (width 0.3556) (layer B.Cu) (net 27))
 (segment (start 168.783 53.594) (end 152.4 69.977) (width 0.3556) (layer B.Cu) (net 20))
 (segment (start 158.422999 90.039801) (end 159.5628 88.9) (width 0.3556) (layer B.Cu) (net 20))
 (segment (start 153.418559 90.039801) (end 158.422999 90.039801) (width 0.3556) (layer B.Cu) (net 20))
 (segment (start 152.4 89.021242) (end 153.418559 90.039801) (width 0.3556) (layer B.Cu) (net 20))
 (segment (start 152.4 69.977) (end 152.4 89.021242) (width 0.3556) (layer B.Cu) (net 20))
 (segment (start 160.792506 87.589706) (end 159.5628 86.36) (width 0.3556) (layer F.Cu) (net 36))
 (segment (start 168.217655 77.816199) (end 166.37 79.663854) (width 0.3556) (layer F.Cu) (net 36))
 (segment (start 169.833801 77.816199) (end 168.217655 77.816199) (width 0.3556) (layer F.Cu) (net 36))
 (segment (start 180.005073 55.868781) (end 180.005073 67.644927) (width 0.3556) (layer F.Cu) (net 36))
 (segment (start 162.56 87.589706) (end 160.792506 87.589706) (width 0.3556) (layer F.Cu) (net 36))
 (segment (start 180.005073 67.644927) (end 169.833801 77.816199) (width 0.3556) (layer F.Cu) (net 36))
 (segment (start 183.457655 52.416199) (end 180.005073 55.868781) (width 0.3556) (layer F.Cu) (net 36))
 (segment (start 185.200801 53.028655) (end 184.588345 52.416199) (width 0.3556) (layer F.Cu) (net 36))
 (segment (start 166.37 83.779706) (end 162.56 87.589706) (width 0.3556) (layer F.Cu) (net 36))
 (segment (start 166.37 79.663854) (end 166.37 83.779706) (width 0.3556) (layer F.Cu) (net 36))
 (segment (start 185.200801 54.956199) (end 185.200801 53.028655) (width 0.3556) (layer F.Cu) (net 36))
 (segment (start 184.588345 52.416199) (end 183.457655 52.416199) (width 0.3556) (layer F.Cu) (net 36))
 (segment (start 184.023 56.134) (end 185.200801 54.956199) (width 0.3556) (layer F.Cu) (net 36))
 (segment (start 167.605199 80.968655) (end 167.605199 83.397601) (width 0.3556) (layer F.Cu) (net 37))
 (segment (start 168.402053 80.171801) (end 167.605199 80.968655) (width 0.3556) (layer F.Cu) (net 37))
 (segment (start 169.348345 80.171801) (end 168.402053 80.171801) (width 0.3556) (layer F.Cu) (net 37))
 (segment (start 167.605199 83.397601) (end 162.1028 88.9) (width 0.3556) (layer F.Cu) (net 37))
 (segment (start 181.592573 67.927573) (end 169.348345 80.171801) (width 0.3556) (layer F.Cu) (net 37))
 (segment (start 181.592573 56.024427) (end 181.592573 67.927573) (width 0.3556) (layer F.Cu) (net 37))
 (segment (start 184.023 53.594) (end 181.592573 56.024427) (width 0.3556) (layer F.Cu) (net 37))
 (segment (start 185.4835 77.5335) (end 184.023 78.994) (width 0.3556) (layer F.Cu) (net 14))
 (segment (start 186.69 76.327) (end 185.4835 77.5335) (width 0.3556) (layer F.Cu) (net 14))
 (segment (start 188.7855 74.2315) (end 187.3885 75.6285) (width 0.3556) (layer F.Cu) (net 14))
 (segment (start 188.7855 52.2605) (end 188.7855 74.2315) (width 0.3556) (layer F.Cu) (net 14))
 (segment (start 187.3885 75.6285) (end 185.4835 77.5335) (width 0.3556) (layer F.Cu) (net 14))
 (segment (start 190.119 50.927) (end 188.7855 52.2605) (width 0.3556) (layer F.Cu) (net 14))
 (segment (start 163.026601 85.436199) (end 162.1028 86.36) (width 0.3556) (layer B.Cu) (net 33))
 (segment (start 169.348345 85.436199) (end 163.026601 85.436199) (width 0.3556) (layer B.Cu) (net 33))
 (segment (start 170.18 84.604544) (end 169.937272 84.847272) (width 0.3556) (layer B.Cu) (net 33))
 (segment (start 169.937272 84.847272) (end 169.348345 85.436199) (width 0.3556) (layer B.Cu) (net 33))
 (segment (start 179.854544 65.382456) (end 184.023 61.214) (width 0.3556) (layer B.Cu) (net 33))
 (segment (start 179.854544 74.93) (end 179.854544 65.382456) (width 0.3556) (layer B.Cu) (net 33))
 (segment (start 169.937272 84.847272) (end 179.854544 74.93) (width 0.3556) (layer B.Cu) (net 33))
 (segment (start 186.924427 52.304427) (end 186.924427 57.550573) (width 0.3556) (layer F.Cu) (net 13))
 (segment (start 185.801 58.674) (end 184.023 58.674) (width 0.3556) (layer F.Cu) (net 13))
 (segment (start 189.529655 49.699199) (end 186.924427 52.304427) (width 0.3556) (layer F.Cu) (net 13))
 (segment (start 191.431199 49.699199) (end 189.529655 49.699199) (width 0.3556) (layer F.Cu) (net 13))
 (segment (start 186.924427 57.550573) (end 185.801 58.674) (width 0.3556) (layer F.Cu) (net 13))
 (segment (start 192.659 50.927) (end 191.431199 49.699199) (width 0.3556) (layer F.Cu) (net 13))
 (segment (start 202.42 69.85) (end 199.39 69.85) (width 0.3556) (layer F.Cu) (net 39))
 (segment (start 196.31 69.85) (end 199.39 69.85) (width 0.3556) (layer F.Cu) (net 39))
 (segment (start 199.39 64.77) (end 202.42 64.77) (width 0.3556) (layer F.Cu) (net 18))
 (segment (start 196.31 64.77) (end 199.39 64.77) (width 0.3556) (layer F.Cu) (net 18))
 (segment (start 199.39 59.69) (end 202.42 59.69) (width 0.3556) (layer F.Cu) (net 40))
 (segment (start 196.31 59.69) (end 199.39 59.69) (width 0.3556) (layer F.Cu) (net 40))
 (segment (start 184.023 71.374) (end 188.976 71.374) (width 0.3556) (layer B.Cu) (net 28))
 (segment (start 188.976 71.374) (end 190.5 69.85) (width 0.3556) (layer B.Cu) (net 28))
 (via (at 190.5 69.85) (size 0.8) (drill 0.4) (layers F.Cu B.Cu) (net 28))
 (segment (start 190.5 69.85) (end 194.31 69.85) (width 0.3556) (layer F.Cu) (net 28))
 (segment (start 184.023 68.834) (end 186.436 68.834) (width 0.3556) (layer B.Cu) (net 19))
 (segment (start 186.436 68.834) (end 189.23 66.04) (width 0.3556) (layer B.Cu) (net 19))
 (segment (start 189.23 66.04) (end 190.5 64.77) (width 0.3556) (layer B.Cu) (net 19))
 (via (at 190.5 64.77) (size 0.8) (drill 0.4) (layers F.Cu B.Cu) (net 19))
 (segment (start 190.5 64.77) (end 194.31 64.77) (width 0.3556) (layer F.Cu) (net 19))
 (segment (start 184.023 66.294) (end 185.166 66.294) (width 0.3556) (layer B.Cu) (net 30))
 (segment (start 185.166 66.294) (end 191.77 59.69) (width 0.3556) (layer B.Cu) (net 30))
 (via (at 191.77 59.69) (size 0.8) (drill 0.4) (layers F.Cu B.Cu) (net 30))
 (segment (start 191.77 59.69) (end 194.31 59.69) (width 0.3556) (layer F.Cu) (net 30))
 (via (at 175.26 76.2) (size 0.8) (drill 0.4) (layers F.Cu B.Cu) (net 15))
 (segment (start 175.26 76.2) (end 172.72 73.66) (width 0.3556) (layer B.Cu) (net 15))
 (segment (start 172.72 65.151) (end 168.783 61.214) (width 0.3556) (layer B.Cu) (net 15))
 (segment (start 172.72 73.66) (end 172.72 65.151) (width 0.3556) (layer B.Cu) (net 15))
 (segment (start 190.34 75.41) (end 190.82 74.93) (width 0.3556) (layer F.Cu) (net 15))
 (segment (start 190.34 78.74) (end 190.34 75.41) (width 0.3556) (layer F.Cu) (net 15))
 (segment (start 189.73304 78.74) (end 188.876 79.59704) (width 0.3556) (layer F.Cu) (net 15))
 (segment (start 190.34 78.74) (end 189.73304 78.74) (width 0.3556) (layer F.Cu) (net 15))
 (segment (start 181.956199 82.896199) (end 175.26 76.2) (width 0.3556) (layer F.Cu) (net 15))
 (segment (start 188.150146 79.15) (end 189.59 79.15) (width 0.3556) (layer F.Cu) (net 15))
 (segment (start 184.403947 82.896199) (end 188.150146 79.15) (width 0.3556) (layer F.Cu) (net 15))
 (segment (start 181.956199 82.896199) (end 184.403947 82.896199) (width 0.3556) (layer F.Cu) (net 15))
 (segment (start 171.069 91.44) (end 168.783 89.154) (width 0.3556) (layer B.Cu) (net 17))
 (segment (start 190.58 91.44) (end 171.069 91.44) (width 0.3556) (layer B.Cu) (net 17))
 (segment (start 190.34 91.2) (end 190.58 91.44) (width 0.3556) (layer F.Cu) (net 17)))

